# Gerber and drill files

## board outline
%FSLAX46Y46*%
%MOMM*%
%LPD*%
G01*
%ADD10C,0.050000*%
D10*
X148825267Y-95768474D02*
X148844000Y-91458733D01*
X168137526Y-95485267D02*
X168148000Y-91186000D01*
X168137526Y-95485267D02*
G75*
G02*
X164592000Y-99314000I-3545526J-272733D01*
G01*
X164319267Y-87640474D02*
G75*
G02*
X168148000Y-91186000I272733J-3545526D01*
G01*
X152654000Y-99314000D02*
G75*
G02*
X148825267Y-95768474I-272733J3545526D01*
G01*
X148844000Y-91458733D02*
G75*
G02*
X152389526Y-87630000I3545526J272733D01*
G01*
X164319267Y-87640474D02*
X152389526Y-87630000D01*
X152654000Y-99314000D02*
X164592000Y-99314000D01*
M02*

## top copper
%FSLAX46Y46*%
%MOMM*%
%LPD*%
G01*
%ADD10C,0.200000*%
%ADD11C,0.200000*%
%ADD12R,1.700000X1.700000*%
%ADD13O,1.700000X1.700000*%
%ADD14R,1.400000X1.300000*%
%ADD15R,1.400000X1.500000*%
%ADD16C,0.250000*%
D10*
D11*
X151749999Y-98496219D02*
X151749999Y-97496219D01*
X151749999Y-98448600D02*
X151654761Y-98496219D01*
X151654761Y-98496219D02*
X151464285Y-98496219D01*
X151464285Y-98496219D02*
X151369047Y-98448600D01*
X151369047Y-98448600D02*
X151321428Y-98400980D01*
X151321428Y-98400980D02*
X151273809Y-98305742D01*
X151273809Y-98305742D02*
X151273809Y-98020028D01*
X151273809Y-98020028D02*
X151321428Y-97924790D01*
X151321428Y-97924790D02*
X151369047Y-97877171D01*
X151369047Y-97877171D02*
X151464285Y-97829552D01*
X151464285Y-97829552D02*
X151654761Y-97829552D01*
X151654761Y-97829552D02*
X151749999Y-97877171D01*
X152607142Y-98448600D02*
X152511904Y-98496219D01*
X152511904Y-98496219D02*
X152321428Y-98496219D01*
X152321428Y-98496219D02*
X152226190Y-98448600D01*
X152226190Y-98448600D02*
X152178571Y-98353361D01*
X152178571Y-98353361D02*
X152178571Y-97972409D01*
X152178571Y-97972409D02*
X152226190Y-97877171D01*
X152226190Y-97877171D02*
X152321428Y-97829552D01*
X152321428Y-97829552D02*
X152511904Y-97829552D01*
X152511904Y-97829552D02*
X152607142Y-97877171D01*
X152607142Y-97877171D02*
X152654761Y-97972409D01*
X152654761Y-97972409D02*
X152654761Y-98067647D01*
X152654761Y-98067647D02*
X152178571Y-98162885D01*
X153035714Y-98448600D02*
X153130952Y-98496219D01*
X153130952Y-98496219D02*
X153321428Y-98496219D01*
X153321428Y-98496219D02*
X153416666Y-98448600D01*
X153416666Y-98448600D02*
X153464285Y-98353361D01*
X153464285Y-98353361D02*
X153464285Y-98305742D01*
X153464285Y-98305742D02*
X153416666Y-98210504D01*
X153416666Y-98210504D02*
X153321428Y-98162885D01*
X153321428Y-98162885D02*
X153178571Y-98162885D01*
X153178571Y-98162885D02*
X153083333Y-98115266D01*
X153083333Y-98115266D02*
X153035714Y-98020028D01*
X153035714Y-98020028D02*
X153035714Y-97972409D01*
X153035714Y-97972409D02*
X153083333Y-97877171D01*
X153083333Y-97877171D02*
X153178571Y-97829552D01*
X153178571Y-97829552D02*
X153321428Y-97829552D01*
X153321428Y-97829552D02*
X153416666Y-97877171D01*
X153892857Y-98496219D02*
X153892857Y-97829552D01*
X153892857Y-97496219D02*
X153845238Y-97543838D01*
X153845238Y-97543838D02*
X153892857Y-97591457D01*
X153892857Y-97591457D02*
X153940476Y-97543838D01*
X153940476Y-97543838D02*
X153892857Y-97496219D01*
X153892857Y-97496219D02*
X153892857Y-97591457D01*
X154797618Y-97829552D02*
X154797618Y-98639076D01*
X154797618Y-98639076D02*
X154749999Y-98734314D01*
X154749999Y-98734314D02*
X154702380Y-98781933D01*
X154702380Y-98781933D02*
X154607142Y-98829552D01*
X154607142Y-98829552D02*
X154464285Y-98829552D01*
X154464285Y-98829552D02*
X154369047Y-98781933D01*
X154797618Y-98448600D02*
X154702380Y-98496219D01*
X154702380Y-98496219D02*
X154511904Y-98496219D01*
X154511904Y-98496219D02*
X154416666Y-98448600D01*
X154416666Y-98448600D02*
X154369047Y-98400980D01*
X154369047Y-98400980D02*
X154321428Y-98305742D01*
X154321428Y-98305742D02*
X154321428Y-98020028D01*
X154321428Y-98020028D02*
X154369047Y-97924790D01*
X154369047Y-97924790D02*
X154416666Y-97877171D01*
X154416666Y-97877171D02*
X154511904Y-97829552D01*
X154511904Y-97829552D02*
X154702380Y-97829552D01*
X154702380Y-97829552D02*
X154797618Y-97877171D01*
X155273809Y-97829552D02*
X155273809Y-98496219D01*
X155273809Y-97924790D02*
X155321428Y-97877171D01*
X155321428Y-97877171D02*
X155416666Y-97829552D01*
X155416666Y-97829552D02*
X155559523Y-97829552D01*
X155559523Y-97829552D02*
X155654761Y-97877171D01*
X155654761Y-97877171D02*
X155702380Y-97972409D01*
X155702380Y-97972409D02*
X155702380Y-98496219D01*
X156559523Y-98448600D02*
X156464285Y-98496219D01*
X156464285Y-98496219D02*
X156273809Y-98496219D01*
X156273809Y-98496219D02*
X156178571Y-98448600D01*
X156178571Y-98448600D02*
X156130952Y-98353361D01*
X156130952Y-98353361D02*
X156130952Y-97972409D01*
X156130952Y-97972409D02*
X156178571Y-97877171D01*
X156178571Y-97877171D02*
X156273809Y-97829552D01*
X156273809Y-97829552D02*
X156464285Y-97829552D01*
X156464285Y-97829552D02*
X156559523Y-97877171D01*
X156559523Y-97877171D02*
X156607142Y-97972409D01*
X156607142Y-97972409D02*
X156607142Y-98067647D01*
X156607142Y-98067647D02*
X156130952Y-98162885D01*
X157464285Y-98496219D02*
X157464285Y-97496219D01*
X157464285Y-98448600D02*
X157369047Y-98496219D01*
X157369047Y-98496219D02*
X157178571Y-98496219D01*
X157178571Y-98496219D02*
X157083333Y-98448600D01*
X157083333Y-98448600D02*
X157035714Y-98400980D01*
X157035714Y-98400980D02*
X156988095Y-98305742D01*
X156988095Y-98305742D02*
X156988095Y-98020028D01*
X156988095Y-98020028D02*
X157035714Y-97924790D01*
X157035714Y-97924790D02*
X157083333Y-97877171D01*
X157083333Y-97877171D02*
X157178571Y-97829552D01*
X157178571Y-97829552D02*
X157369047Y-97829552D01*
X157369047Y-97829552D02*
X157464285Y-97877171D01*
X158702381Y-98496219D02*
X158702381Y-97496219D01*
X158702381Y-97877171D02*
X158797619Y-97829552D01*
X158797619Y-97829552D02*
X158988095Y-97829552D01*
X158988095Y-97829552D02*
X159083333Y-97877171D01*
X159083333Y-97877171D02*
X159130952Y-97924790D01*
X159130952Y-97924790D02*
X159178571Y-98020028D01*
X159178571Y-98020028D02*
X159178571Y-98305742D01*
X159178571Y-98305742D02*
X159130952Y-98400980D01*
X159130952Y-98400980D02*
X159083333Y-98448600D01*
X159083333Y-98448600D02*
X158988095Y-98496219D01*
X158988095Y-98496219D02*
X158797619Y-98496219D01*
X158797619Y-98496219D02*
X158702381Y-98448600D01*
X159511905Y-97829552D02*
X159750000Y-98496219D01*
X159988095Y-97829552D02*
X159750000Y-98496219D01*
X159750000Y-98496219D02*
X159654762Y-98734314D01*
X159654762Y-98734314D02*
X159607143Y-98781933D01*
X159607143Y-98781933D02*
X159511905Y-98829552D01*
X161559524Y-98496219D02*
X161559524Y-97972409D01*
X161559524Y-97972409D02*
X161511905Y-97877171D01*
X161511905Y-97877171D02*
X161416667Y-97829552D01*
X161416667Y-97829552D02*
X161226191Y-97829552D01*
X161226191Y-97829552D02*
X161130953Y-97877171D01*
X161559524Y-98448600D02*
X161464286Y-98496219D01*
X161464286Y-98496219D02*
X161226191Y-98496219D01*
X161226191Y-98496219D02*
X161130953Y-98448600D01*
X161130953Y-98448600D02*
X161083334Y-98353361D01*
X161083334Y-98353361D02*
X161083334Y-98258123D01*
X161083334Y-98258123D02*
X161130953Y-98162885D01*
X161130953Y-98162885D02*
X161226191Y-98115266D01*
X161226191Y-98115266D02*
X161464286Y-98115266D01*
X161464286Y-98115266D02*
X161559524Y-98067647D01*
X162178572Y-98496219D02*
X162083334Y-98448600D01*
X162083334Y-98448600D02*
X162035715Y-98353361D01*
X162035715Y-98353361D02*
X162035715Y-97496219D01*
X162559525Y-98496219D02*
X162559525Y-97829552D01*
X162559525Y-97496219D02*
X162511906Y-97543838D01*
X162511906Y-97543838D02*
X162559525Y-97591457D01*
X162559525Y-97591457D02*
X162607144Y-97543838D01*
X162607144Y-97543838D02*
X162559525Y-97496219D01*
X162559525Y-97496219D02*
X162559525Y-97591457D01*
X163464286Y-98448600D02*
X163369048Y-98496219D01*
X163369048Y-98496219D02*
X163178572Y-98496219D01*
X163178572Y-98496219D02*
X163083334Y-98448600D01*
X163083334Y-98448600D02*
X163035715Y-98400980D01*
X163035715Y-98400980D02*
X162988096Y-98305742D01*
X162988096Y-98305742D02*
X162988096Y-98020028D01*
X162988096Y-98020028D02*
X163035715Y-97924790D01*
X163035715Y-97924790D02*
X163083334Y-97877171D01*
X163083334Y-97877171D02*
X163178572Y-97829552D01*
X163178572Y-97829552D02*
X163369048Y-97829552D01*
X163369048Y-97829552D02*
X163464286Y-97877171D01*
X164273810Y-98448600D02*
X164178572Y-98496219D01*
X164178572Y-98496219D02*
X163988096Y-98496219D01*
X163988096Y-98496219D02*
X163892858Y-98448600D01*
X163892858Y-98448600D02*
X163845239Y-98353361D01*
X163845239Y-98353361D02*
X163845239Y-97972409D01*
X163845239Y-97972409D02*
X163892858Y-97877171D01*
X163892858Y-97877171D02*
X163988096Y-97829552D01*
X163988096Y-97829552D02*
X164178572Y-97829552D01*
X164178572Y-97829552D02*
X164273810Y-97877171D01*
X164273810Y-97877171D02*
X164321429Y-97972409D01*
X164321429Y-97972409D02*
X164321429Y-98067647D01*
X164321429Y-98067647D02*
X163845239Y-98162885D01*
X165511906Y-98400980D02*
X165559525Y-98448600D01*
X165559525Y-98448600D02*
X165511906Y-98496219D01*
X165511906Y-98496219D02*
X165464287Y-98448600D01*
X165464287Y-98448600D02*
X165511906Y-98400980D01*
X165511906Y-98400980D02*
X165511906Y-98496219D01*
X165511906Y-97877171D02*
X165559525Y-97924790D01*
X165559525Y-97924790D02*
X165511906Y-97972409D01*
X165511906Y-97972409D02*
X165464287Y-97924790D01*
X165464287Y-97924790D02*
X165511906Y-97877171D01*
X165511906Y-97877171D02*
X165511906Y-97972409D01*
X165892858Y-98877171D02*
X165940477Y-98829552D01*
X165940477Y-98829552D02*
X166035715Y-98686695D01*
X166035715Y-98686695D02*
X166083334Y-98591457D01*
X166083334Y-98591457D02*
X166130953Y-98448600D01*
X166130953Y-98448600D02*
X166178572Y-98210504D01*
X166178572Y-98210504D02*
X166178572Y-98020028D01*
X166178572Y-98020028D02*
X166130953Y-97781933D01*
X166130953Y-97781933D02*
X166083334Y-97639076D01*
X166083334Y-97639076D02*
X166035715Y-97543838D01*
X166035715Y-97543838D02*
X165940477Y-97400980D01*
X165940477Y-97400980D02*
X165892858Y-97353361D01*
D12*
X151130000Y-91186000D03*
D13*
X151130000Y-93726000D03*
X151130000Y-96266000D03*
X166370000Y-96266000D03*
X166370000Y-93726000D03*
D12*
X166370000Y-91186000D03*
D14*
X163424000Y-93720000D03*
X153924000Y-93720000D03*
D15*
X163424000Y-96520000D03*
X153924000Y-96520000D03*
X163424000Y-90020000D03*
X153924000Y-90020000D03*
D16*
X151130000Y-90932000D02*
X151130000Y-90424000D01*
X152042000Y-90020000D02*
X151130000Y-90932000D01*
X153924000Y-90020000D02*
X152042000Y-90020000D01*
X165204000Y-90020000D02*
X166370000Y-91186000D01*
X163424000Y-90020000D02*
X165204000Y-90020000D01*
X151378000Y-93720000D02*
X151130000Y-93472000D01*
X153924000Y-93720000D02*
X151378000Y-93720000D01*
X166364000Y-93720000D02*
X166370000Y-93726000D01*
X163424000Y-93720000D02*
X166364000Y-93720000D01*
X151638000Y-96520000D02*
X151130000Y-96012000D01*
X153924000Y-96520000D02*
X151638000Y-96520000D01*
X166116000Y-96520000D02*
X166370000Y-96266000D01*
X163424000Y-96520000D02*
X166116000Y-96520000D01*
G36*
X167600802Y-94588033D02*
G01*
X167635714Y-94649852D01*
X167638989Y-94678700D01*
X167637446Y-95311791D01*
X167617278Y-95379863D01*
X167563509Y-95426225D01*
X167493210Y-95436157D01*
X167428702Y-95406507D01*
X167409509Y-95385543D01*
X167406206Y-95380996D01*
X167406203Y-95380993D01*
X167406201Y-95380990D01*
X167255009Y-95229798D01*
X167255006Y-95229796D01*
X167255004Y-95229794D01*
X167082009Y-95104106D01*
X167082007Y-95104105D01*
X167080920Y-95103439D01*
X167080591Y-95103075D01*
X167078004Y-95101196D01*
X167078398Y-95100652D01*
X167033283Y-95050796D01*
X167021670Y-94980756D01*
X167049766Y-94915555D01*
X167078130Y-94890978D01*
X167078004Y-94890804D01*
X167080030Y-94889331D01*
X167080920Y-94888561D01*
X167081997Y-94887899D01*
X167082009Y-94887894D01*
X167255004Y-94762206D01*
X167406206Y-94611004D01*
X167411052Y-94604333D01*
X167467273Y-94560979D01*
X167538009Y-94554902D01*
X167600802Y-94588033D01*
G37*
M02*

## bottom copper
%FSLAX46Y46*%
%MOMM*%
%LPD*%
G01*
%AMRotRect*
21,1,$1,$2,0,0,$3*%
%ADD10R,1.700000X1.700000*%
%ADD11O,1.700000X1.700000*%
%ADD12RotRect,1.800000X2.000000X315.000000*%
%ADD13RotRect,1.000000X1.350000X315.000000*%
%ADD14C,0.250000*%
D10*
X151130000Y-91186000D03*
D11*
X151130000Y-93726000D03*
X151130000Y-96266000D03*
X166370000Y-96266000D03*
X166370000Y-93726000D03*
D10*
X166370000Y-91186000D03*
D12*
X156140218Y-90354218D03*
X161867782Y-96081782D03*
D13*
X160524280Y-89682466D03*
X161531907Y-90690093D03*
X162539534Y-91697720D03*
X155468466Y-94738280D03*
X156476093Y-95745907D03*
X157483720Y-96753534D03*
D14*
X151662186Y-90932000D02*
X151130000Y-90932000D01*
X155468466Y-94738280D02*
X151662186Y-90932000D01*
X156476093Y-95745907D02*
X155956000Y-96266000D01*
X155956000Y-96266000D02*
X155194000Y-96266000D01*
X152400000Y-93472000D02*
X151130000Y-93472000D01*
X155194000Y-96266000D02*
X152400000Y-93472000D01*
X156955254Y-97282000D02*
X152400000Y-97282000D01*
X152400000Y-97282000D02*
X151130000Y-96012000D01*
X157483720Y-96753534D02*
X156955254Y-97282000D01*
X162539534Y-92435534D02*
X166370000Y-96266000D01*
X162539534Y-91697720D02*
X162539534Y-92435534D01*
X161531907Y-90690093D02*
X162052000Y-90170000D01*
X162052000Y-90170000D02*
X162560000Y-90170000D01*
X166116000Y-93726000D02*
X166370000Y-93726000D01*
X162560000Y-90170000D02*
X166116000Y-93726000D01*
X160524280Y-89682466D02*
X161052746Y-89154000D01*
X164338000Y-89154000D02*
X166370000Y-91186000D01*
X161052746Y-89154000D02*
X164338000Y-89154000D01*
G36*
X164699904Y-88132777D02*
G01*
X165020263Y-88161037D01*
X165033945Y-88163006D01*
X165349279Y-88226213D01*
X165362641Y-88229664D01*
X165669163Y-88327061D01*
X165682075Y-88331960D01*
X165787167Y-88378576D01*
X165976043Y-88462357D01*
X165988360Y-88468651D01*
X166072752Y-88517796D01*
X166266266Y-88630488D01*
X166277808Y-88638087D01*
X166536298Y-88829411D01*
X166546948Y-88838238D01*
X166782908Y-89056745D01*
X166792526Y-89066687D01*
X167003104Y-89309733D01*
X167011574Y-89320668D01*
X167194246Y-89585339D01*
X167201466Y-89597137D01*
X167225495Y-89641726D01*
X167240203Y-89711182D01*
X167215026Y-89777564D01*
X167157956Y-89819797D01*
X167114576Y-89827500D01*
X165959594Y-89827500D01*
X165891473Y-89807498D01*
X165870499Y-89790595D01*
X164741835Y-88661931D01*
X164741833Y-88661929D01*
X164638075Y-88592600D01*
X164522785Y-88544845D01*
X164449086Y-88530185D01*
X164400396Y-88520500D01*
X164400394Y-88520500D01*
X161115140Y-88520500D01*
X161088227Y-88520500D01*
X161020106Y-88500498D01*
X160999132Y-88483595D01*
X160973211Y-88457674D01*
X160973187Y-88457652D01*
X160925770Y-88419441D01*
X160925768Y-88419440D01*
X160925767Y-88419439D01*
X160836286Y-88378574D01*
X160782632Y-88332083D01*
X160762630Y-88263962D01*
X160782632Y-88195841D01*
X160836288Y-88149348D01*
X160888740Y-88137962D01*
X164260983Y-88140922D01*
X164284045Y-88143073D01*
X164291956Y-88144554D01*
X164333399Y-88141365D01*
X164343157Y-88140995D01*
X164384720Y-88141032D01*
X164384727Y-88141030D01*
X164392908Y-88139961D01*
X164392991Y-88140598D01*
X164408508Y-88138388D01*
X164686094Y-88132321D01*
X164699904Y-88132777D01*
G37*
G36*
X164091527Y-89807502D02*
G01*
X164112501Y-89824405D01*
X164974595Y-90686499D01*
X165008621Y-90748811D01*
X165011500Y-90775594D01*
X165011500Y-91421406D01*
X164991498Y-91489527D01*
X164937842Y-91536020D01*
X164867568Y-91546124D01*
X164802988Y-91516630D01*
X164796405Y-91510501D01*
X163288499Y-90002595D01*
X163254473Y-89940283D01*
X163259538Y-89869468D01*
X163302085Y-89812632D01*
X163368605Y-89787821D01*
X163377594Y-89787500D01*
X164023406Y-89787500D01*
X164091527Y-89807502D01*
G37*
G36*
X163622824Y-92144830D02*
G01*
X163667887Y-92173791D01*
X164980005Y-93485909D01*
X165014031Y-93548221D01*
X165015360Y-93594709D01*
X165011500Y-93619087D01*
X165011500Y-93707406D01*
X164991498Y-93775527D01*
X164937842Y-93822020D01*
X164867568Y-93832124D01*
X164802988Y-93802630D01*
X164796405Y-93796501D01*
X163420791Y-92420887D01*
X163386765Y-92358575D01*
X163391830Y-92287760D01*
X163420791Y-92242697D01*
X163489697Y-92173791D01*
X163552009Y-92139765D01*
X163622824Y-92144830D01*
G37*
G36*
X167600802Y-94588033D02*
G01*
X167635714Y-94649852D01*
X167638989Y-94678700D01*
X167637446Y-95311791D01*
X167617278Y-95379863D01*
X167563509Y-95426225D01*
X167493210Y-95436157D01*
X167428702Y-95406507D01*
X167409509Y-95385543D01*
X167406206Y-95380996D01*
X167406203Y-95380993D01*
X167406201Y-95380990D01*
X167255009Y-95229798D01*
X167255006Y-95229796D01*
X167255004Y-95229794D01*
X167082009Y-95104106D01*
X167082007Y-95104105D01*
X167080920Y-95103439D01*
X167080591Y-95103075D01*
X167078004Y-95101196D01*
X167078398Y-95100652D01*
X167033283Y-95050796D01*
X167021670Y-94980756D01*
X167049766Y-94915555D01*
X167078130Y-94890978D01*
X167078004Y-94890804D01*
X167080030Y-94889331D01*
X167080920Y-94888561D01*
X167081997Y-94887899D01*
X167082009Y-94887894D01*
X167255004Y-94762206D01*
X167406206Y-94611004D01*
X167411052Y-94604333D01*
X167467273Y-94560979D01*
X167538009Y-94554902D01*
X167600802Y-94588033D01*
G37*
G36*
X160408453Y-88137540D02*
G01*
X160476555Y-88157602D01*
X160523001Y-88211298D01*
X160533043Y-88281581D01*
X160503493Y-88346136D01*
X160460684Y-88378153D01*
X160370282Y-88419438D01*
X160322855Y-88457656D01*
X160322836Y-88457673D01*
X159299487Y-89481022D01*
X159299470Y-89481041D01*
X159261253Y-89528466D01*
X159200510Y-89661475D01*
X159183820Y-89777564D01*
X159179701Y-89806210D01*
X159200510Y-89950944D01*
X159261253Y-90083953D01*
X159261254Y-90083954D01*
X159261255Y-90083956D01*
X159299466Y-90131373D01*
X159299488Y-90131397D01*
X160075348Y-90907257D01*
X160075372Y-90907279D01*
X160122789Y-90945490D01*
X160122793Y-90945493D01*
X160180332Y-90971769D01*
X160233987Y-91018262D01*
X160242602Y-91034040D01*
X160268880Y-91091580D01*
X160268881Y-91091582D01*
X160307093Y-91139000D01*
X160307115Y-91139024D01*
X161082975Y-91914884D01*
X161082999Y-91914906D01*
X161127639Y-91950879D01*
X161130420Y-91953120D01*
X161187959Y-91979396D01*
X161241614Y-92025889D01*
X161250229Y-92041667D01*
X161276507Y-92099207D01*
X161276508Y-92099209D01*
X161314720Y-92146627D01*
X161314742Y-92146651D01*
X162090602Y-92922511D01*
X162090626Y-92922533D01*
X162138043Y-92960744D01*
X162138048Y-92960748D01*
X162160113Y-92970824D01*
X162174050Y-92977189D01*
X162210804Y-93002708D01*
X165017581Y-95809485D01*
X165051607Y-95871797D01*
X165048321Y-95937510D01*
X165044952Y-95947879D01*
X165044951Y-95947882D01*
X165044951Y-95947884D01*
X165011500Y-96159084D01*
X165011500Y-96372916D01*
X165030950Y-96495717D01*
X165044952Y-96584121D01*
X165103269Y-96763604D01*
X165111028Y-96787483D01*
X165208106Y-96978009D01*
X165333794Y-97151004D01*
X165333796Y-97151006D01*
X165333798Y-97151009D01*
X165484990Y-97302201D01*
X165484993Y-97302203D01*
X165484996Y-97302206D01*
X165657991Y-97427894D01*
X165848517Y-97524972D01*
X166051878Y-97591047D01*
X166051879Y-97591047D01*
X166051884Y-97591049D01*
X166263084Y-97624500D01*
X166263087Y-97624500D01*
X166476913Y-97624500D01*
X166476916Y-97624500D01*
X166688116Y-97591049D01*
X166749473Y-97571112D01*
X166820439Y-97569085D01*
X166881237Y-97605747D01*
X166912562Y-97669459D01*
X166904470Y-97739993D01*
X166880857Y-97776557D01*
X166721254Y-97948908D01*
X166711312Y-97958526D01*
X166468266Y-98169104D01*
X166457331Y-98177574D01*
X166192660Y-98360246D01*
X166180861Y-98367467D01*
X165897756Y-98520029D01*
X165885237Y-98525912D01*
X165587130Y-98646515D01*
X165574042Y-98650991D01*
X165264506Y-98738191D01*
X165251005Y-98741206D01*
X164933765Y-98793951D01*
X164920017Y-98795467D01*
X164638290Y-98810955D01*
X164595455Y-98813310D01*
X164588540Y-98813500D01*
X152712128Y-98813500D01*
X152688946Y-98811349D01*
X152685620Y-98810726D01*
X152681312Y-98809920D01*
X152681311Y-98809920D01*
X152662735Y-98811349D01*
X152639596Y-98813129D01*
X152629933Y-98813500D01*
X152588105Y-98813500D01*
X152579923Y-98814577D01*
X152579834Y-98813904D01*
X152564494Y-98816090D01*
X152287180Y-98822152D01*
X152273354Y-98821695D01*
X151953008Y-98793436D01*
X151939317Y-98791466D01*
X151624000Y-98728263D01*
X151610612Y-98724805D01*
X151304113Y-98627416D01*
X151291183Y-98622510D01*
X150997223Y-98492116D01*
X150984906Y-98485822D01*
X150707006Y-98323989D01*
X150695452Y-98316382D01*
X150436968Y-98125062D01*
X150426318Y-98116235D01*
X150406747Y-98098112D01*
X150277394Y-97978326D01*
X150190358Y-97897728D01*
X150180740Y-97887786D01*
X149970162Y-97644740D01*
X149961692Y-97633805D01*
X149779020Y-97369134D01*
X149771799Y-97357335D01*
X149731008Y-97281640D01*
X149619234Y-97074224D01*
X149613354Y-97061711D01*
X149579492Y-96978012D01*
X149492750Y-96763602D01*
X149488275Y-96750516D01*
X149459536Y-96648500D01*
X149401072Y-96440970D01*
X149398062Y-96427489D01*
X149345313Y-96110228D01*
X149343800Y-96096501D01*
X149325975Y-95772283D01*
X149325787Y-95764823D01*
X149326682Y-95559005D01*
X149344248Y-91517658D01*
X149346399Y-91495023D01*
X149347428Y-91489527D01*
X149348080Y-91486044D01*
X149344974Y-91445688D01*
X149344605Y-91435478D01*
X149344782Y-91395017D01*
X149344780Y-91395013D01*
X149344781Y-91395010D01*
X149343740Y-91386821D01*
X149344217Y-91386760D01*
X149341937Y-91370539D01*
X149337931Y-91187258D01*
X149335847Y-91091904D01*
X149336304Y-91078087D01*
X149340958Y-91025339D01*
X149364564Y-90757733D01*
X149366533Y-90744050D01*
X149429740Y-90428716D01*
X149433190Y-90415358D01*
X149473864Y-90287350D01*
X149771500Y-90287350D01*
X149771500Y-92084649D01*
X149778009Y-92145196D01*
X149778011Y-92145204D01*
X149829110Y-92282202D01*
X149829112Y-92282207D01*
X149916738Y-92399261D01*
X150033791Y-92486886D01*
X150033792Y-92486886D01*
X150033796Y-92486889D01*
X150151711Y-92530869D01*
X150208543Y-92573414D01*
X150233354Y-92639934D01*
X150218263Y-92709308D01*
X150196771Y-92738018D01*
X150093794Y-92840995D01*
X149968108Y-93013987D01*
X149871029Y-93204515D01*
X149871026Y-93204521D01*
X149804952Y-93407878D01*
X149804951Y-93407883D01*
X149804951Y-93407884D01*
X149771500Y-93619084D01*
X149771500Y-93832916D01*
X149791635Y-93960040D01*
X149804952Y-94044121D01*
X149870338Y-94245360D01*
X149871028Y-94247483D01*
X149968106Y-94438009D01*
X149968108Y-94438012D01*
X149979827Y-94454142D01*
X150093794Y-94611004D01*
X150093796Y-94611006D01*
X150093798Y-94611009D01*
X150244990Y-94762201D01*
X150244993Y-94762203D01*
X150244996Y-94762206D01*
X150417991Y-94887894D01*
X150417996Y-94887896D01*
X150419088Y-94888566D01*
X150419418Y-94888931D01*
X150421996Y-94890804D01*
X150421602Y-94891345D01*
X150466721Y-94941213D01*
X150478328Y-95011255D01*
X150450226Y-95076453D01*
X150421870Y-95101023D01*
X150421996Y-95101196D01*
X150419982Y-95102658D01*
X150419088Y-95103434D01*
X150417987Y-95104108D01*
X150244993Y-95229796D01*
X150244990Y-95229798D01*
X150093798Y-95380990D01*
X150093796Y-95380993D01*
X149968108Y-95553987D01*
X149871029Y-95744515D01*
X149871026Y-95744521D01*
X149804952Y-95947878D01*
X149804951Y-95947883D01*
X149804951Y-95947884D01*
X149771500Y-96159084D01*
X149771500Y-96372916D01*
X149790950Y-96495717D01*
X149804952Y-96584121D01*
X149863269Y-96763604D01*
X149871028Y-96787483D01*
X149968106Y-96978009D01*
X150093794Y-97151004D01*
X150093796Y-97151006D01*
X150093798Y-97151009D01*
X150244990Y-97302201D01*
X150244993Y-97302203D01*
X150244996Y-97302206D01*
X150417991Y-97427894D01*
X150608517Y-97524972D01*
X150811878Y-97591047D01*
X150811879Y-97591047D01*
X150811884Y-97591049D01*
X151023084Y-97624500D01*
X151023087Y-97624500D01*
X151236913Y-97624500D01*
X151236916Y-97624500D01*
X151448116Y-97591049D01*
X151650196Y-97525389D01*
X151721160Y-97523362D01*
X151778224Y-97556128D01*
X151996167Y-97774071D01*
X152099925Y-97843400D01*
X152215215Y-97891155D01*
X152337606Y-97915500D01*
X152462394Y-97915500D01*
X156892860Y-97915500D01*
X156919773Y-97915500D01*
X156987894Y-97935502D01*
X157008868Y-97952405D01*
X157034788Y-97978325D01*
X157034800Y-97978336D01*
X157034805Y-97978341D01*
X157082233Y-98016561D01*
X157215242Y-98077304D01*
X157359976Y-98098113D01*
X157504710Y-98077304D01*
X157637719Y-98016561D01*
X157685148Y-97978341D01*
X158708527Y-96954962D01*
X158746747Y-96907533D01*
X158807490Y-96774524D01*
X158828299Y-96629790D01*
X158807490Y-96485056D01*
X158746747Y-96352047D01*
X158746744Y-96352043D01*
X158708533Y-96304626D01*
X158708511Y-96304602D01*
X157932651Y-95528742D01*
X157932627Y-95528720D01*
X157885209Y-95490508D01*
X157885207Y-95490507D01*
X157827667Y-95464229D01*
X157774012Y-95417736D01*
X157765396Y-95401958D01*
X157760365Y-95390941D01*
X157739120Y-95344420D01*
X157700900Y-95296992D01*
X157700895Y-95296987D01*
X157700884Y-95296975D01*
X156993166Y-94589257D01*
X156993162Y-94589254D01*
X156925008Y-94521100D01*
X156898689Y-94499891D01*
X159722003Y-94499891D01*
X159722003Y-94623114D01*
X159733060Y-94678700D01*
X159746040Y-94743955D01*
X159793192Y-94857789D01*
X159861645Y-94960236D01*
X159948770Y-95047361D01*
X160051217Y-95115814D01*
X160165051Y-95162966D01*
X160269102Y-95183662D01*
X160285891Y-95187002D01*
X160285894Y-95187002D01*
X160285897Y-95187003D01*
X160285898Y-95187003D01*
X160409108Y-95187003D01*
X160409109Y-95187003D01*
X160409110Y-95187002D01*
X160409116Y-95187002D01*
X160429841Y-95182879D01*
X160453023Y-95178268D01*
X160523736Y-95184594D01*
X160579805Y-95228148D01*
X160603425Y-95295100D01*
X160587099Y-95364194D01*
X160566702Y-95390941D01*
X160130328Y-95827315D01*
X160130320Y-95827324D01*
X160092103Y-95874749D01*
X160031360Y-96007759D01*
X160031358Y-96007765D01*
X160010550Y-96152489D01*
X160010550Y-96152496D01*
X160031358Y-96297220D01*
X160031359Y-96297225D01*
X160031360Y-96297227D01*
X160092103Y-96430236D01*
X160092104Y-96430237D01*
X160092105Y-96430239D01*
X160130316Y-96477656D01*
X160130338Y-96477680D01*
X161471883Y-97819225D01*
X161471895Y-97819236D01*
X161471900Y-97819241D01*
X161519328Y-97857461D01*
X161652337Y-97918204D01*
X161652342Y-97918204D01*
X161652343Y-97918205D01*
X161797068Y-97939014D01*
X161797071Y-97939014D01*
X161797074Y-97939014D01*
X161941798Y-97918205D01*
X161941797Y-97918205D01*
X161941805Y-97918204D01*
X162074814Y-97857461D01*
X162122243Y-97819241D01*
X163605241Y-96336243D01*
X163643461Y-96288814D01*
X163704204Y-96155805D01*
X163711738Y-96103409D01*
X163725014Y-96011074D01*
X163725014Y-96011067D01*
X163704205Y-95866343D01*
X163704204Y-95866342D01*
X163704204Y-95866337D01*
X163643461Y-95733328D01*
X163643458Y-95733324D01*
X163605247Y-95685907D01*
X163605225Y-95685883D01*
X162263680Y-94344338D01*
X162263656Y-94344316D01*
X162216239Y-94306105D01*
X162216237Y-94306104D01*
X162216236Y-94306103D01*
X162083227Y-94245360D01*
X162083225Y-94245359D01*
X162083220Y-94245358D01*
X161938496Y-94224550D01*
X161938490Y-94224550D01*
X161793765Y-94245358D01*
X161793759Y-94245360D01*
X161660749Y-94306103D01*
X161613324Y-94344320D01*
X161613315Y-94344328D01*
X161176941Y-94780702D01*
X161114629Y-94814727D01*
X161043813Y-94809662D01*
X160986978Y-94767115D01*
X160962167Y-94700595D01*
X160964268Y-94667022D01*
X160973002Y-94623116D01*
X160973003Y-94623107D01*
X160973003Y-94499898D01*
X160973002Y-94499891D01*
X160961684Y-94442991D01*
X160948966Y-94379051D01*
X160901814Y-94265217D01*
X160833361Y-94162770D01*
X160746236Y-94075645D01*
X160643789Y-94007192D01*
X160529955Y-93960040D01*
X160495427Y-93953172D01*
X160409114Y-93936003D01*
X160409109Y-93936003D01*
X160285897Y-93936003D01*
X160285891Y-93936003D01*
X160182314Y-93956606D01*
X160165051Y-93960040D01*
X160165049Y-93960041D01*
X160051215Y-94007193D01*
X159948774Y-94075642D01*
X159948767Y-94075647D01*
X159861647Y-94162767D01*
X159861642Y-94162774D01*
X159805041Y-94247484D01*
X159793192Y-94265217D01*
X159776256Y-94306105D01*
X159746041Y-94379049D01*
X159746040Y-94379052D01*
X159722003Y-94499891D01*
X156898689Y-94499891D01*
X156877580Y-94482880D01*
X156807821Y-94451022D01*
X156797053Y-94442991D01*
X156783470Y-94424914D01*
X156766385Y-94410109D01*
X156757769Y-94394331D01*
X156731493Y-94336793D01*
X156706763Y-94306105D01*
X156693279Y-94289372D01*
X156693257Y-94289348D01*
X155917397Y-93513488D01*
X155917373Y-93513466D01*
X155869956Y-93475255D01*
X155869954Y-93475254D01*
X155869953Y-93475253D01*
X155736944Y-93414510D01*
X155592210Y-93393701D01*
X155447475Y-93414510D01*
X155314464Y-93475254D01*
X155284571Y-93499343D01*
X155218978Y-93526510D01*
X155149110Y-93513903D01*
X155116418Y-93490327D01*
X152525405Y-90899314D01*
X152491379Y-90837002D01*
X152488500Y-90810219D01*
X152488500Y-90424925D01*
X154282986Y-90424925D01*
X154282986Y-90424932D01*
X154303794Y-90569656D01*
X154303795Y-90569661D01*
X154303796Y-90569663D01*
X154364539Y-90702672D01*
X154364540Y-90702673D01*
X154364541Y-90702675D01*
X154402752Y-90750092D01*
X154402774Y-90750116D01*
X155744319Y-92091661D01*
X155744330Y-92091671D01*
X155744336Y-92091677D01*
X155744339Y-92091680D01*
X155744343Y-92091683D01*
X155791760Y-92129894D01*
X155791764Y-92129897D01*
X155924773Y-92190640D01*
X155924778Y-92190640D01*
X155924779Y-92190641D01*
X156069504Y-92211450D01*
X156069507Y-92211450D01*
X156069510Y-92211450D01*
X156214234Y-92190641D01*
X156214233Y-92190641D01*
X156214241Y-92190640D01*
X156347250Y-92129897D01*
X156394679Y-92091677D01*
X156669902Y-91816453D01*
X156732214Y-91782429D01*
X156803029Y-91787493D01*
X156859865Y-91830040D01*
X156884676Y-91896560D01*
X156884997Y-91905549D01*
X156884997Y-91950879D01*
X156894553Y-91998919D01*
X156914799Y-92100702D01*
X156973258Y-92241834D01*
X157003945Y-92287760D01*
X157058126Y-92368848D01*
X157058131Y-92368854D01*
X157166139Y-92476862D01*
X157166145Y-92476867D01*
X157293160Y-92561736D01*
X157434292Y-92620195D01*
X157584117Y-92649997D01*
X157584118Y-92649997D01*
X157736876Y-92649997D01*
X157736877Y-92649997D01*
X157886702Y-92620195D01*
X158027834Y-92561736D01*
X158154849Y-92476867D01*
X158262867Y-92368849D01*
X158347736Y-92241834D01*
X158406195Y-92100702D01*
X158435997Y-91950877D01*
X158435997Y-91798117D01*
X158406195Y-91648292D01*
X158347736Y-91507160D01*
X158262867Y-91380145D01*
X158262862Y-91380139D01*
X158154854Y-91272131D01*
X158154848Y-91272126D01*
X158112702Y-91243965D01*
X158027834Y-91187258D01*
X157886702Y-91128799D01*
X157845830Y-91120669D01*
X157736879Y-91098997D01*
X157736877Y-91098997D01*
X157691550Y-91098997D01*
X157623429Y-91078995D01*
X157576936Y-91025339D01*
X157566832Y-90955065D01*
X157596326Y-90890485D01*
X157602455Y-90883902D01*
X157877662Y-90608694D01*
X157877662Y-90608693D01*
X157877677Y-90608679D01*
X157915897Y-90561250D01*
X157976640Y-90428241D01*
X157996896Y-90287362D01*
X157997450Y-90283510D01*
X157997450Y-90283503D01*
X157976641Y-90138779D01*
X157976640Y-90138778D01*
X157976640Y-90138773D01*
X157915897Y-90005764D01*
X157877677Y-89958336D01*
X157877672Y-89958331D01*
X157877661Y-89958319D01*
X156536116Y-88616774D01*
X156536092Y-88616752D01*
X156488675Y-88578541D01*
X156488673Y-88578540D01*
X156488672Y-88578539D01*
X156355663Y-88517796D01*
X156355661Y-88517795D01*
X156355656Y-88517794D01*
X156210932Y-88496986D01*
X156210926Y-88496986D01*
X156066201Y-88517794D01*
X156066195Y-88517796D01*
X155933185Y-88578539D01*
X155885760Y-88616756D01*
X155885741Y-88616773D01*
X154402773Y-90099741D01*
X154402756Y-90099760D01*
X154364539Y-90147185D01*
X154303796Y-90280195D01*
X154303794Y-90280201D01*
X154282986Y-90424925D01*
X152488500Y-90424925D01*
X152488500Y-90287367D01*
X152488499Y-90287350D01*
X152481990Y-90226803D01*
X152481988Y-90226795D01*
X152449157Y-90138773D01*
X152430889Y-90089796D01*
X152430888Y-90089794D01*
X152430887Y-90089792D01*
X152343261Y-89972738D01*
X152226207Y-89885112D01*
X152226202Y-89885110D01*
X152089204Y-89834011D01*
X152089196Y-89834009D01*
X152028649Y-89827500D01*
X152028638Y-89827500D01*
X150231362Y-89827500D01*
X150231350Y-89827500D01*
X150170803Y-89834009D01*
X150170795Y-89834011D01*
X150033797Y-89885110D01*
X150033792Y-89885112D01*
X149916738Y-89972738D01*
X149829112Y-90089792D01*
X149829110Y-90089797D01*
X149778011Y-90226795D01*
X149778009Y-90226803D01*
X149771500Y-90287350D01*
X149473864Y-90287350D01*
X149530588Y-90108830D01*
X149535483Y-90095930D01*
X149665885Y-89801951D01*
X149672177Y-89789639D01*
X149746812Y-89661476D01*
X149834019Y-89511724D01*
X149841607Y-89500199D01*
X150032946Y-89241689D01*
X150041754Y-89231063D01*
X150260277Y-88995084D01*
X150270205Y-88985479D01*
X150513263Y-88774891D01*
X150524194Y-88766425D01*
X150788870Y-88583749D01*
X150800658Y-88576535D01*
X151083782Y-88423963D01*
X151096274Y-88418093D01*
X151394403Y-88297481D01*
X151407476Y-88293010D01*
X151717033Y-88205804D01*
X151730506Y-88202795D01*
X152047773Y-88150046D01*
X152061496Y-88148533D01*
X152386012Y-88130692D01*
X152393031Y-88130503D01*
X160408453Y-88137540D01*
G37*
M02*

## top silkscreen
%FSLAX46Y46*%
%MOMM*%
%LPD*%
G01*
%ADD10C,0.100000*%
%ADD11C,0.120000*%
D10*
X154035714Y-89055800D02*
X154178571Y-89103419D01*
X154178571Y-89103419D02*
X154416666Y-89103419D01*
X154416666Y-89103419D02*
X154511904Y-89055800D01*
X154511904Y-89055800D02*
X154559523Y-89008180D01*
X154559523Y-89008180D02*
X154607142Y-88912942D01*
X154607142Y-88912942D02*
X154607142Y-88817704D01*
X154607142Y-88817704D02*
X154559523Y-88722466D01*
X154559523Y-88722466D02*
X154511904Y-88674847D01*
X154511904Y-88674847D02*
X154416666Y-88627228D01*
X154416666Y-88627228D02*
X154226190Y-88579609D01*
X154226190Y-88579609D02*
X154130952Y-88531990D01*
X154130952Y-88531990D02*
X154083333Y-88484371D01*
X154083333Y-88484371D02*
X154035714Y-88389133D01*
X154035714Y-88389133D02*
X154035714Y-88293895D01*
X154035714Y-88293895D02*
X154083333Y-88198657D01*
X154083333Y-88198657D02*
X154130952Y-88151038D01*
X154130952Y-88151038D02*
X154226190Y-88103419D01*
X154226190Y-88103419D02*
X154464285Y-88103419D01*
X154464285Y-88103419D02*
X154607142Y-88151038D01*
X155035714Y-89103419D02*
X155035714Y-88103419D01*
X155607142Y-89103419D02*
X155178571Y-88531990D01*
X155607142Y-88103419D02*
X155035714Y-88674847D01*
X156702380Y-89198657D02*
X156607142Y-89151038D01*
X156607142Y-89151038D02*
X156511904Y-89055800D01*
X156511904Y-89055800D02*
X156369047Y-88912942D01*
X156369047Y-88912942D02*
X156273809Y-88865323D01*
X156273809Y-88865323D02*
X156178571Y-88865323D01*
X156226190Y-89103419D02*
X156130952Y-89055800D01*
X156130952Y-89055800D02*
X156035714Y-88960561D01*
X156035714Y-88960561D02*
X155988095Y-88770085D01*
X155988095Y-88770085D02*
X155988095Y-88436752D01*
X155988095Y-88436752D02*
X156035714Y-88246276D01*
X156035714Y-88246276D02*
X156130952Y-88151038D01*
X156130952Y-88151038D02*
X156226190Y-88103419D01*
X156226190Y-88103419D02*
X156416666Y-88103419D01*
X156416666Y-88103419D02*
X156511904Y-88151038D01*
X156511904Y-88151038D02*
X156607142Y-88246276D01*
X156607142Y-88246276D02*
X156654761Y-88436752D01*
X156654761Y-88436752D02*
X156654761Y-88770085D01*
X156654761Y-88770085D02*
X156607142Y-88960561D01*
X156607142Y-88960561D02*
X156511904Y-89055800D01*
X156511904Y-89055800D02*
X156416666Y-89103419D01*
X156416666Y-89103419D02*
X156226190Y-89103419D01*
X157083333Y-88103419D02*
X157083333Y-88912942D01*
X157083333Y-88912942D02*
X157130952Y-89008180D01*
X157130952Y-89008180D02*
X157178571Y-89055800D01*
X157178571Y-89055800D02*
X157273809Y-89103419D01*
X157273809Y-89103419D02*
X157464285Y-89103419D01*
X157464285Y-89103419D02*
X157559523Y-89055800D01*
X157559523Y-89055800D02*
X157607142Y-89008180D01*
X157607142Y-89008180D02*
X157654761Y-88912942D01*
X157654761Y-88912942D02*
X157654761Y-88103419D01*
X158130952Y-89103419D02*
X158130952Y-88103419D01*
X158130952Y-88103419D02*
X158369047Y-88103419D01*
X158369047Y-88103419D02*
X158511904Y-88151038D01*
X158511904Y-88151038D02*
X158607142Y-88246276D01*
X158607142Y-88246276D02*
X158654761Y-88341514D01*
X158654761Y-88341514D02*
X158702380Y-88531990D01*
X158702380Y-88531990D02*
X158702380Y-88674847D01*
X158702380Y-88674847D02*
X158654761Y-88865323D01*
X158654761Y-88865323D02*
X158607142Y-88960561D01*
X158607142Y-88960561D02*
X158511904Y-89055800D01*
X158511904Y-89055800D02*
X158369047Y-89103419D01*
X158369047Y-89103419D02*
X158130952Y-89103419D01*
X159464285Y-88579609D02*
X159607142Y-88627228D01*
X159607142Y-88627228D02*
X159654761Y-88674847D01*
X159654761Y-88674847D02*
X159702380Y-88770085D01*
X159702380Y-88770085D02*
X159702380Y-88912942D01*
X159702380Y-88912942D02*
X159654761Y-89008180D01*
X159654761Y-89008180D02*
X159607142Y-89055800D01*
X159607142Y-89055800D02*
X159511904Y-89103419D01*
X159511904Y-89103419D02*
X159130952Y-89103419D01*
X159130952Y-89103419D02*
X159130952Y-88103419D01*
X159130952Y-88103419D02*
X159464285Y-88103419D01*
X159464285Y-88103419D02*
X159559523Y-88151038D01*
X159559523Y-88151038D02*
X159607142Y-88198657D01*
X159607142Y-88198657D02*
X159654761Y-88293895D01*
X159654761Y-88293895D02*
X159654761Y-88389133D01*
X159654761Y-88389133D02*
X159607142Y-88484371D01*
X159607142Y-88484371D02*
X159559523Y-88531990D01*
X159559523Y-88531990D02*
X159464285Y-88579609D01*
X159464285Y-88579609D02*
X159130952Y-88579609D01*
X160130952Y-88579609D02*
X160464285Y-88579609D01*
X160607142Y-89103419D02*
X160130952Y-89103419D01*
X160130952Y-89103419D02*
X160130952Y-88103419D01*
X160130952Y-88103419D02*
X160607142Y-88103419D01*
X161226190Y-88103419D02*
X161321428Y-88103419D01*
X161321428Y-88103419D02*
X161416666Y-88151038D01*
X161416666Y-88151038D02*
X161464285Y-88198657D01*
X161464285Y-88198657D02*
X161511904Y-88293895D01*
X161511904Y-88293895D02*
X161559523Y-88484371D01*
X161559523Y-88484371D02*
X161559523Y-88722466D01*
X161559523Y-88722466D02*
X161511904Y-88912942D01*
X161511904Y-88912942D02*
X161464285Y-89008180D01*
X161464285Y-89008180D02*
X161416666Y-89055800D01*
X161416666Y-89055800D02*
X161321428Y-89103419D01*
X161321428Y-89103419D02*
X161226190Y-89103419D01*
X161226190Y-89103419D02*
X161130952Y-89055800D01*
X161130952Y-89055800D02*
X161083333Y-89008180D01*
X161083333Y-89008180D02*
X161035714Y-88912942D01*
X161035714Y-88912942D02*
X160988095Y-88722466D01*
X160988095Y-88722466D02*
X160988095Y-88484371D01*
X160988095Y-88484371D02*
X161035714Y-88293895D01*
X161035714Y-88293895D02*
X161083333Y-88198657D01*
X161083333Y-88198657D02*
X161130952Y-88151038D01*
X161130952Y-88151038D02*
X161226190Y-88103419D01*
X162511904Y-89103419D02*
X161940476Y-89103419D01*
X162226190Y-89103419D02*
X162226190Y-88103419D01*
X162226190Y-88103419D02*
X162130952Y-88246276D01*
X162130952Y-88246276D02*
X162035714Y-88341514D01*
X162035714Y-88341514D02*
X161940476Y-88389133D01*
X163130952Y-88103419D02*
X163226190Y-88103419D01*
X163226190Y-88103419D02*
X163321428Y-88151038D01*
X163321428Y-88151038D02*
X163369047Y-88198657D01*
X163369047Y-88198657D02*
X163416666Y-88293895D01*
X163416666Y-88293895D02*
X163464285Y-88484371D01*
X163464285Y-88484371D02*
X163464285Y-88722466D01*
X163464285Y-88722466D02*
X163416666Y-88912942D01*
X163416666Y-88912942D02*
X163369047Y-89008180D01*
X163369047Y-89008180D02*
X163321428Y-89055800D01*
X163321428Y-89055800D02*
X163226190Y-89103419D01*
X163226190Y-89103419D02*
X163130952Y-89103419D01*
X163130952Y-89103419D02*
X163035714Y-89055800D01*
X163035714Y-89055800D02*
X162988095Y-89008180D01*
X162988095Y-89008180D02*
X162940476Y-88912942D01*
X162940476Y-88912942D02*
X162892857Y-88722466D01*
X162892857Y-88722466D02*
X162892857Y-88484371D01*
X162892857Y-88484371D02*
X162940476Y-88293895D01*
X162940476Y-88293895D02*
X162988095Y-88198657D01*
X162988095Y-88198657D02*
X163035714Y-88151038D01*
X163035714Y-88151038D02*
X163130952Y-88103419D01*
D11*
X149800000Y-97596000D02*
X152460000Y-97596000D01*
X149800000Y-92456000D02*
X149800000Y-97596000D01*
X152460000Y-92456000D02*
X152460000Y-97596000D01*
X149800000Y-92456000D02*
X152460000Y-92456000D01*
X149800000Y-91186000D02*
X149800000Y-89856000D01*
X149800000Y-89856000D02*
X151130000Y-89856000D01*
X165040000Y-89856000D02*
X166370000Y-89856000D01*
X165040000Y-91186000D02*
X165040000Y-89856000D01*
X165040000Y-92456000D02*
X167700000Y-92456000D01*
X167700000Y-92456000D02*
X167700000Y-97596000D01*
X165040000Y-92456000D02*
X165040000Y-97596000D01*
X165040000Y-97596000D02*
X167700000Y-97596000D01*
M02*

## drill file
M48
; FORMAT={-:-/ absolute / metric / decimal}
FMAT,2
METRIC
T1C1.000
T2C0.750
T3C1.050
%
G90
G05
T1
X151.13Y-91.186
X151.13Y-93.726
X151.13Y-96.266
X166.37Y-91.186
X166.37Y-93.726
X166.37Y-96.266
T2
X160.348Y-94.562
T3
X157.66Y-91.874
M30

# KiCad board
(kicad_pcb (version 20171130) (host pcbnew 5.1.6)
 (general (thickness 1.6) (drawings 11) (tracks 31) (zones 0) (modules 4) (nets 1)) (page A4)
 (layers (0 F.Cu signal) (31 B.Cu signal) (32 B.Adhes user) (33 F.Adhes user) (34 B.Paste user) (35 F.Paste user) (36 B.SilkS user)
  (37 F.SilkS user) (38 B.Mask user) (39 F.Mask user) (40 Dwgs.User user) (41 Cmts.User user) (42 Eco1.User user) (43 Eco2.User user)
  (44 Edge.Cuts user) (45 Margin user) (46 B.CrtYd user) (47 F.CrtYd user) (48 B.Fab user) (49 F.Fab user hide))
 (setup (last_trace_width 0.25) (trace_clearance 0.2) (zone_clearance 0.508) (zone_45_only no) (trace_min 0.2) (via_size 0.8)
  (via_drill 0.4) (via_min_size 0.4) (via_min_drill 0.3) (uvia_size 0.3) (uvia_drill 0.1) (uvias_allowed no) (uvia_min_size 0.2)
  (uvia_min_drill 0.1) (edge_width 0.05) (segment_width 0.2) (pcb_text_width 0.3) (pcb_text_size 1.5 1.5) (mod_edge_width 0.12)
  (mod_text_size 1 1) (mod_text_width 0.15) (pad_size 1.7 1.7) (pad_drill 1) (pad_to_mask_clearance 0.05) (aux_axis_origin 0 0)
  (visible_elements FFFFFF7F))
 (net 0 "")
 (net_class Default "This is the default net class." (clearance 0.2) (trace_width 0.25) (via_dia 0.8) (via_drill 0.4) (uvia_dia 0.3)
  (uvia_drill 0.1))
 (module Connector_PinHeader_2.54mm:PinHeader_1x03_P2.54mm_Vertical (layer F.Cu) (at 151.13 91.186)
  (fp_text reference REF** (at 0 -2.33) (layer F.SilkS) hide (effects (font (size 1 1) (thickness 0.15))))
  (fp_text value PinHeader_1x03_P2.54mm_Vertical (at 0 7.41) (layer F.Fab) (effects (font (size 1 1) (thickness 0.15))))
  (fp_line (start -1.33 6.41) (end 1.33 6.41) (layer F.SilkS) (width 0.12))
  (fp_line (start -1.33 1.27) (end -1.33 6.41) (layer F.SilkS) (width 0.12))
  (fp_line (start 1.33 1.27) (end 1.33 6.41) (layer F.SilkS) (width 0.12))
  (fp_line (start -1.33 1.27) (end 1.33 1.27) (layer F.SilkS) (width 0.12))
  (fp_line (start -1.33 0) (end -1.33 -1.33) (layer F.SilkS) (width 0.12))
  (fp_line (start -1.33 -1.33) (end 0 -1.33) (layer F.SilkS) (width 0.12))
  (pad 1 thru_hole rect (at 0 0) (size 1.7 1.7) (drill 1) (layers *.Cu *.Mask))
  (pad 2 thru_hole oval (at 0 2.54) (size 1.7 1.7) (drill 1) (layers *.Cu *.Mask))
  (pad 3 thru_hole oval (at 0 5.08) (size 1.7 1.7) (drill 1) (layers *.Cu *.Mask)))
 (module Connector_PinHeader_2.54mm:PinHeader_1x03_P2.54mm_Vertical (layer F.Cu) (at 166.37 91.186)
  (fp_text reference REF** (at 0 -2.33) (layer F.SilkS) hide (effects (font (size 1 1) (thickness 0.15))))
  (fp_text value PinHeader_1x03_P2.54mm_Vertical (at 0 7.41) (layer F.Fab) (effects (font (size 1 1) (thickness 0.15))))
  (fp_line (start -1.33 -1.33) (end 0 -1.33) (layer F.SilkS) (width 0.12))
  (fp_line (start -1.33 0) (end -1.33 -1.33) (layer F.SilkS) (width 0.12))
  (fp_line (start -1.33 1.27) (end 1.33 1.27) (layer F.SilkS) (width 0.12))
  (fp_line (start 1.33 1.27) (end 1.33 6.41) (layer F.SilkS) (width 0.12))
  (fp_line (start -1.33 1.27) (end -1.33 6.41) (layer F.SilkS) (width 0.12))
  (fp_line (start -1.33 6.41) (end 1.33 6.41) (layer F.SilkS) (width 0.12))
  (pad 3 thru_hole oval (at 0 5.08) (size 1.7 1.7) (drill 1) (layers *.Cu *.Mask))
  (pad 2 thru_hole oval (at 0 2.54) (size 1.7 1.7) (drill 1) (layers *.Cu *.Mask))
  (pad 1 thru_hole rect (at 0 0) (size 1.7 1.7) (drill 1) (layers *.Cu *.Mask)))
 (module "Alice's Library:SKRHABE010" (layer B.Cu) (at 159.004 93.218 45)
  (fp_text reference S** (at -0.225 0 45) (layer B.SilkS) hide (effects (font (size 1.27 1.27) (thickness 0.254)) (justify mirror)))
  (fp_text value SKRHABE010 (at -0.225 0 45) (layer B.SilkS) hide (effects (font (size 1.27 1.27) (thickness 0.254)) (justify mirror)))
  (pad GB2 np_thru_hole circle (at 0 -1.9 45) (size 1.05 0) (drill 1.05) (layers *.Cu *.Mask))
  (pad GB1 np_thru_hole circle (at 0 1.9 45) (size 0.75 0) (drill 0.75) (layers *.Cu *.Mask))
  (pad 8 smd rect (at 0 -4.05 315) (size 1.8 2) (layers B.Cu B.Paste B.Mask))
  (pad 7 smd rect (at 0 4.05 315) (size 1.8 2) (layers B.Cu B.Paste B.Mask))
  (pad 6 smd rect (at 3.575 -1.425 315) (size 1 1.35) (layers B.Cu B.Paste B.Mask))
  (pad 5 smd rect (at 3.575 0 315) (size 1 1.35) (layers B.Cu B.Paste B.Mask))
  (pad 4 smd rect (at 3.575 1.425 315) (size 1 1.35) (layers B.Cu B.Paste B.Mask))
  (pad 3 smd rect (at -3.575 -1.425 315) (size 1 1.35) (layers B.Cu B.Paste B.Mask))
  (pad 2 smd rect (at -3.575 0 315) (size 1 1.35) (layers B.Cu B.Paste B.Mask))
  (pad 1 smd rect (at -3.575 1.425 315) (size 1 1.35) (layers B.Cu B.Paste B.Mask)))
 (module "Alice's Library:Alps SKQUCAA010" (layer F.Cu) (at 153.924 90.02)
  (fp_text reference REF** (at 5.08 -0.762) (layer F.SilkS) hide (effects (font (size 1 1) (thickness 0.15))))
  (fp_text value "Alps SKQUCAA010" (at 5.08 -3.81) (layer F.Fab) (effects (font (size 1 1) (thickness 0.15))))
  (pad 5 smd rect (at 9.5 3.7) (size 1.4 1.3) (layers F.Cu F.Paste F.Mask))
  (pad 2 smd rect (at 0 3.7) (size 1.4 1.3) (layers F.Cu F.Paste F.Mask))
  (pad 4 smd rect (at 9.5 6.5) (size 1.4 1.5) (layers F.Cu F.Paste F.Mask))
  (pad 3 smd rect (at 0 6.5) (size 1.4 1.5) (layers F.Cu F.Paste F.Mask))
  (pad 6 smd rect (at 9.5 0) (size 1.4 1.5) (layers F.Cu F.Paste F.Mask))
  (pad 1 smd rect (at 0 0) (size 1.4 1.5) (layers F.Cu F.Paste F.Mask)))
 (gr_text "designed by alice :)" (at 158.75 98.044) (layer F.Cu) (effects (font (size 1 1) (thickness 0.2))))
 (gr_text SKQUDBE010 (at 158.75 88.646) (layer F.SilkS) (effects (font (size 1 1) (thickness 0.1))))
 (gr_line (start 148.825267 95.768474) (end 148.844 91.458733) (layer Edge.Cuts) (width 0.05))
 (gr_line (start 168.137526 95.485267) (end 168.148 91.186) (layer Edge.Cuts) (width 0.05))
 (gr_arc (start 164.592 95.758) (end 164.592 99.314) (angle -94.39870535) (layer Edge.Cuts) (width 0.05))
 (gr_arc (start 164.592 91.186) (end 168.148 91.186) (angle -94.39870535) (layer Edge.Cuts) (width 0.05))
 (gr_arc (start 152.381267 95.768474) (end 148.825267 95.768474) (angle -94.39870535) (layer Edge.Cuts) (width 0.05))
 (gr_arc (start 152.389526 91.186) (end 152.389526 87.63) (angle -94.39870535) (layer Edge.Cuts) (width 0.05))
 (gr_line (start 164.319267 87.640474) (end 152.389526 87.63) (layer Edge.Cuts) (width 0.05))
 (gr_line (start 152.654 99.314) (end 164.592 99.314) (layer Edge.Cuts) (width 0.05))
 (segment (start 151.13 90.932) (end 151.13 90.424) (width 0.25) (layer F.Cu) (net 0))
 (segment (start 152.042 90.02) (end 151.13 90.932) (width 0.25) (layer F.Cu) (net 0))
 (segment (start 153.924 90.02) (end 152.042 90.02) (width 0.25) (layer F.Cu) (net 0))
 (segment (start 165.204 90.02) (end 166.37 91.186) (width 0.25) (layer F.Cu) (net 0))
 (segment (start 163.424 90.02) (end 165.204 90.02) (width 0.25) (layer F.Cu) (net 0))
 (segment (start 151.378 93.72) (end 151.13 93.472) (width 0.25) (layer F.Cu) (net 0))
 (segment (start 153.924 93.72) (end 151.378 93.72) (width 0.25) (layer F.Cu) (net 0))
 (segment (start 166.364 93.72) (end 166.37 93.726) (width 0.25) (layer F.Cu) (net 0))
 (segment (start 163.424 93.72) (end 166.364 93.72) (width 0.25) (layer F.Cu) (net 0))
 (segment (start 151.638 96.52) (end 151.13 96.012) (width 0.25) (layer F.Cu) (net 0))
 (segment (start 153.924 96.52) (end 151.638 96.52) (width 0.25) (layer F.Cu) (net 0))
 (segment (start 166.116 96.52) (end 166.37 96.266) (width 0.25) (layer F.Cu) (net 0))
 (segment (start 163.424 96.52) (end 166.116 96.52) (width 0.25) (layer F.Cu) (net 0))
 (segment (start 151.662186 90.932) (end 151.13 90.932) (width 0.25) (layer B.Cu) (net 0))
 (segment (start 155.468466 94.73828) (end 151.662186 90.932) (width 0.25) (layer B.Cu) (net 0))
 (segment (start 156.476093 95.745907) (end 155.956 96.266) (width 0.25) (layer B.Cu) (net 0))
 (segment (start 155.956 96.266) (end 155.194 96.266) (width 0.25) (layer B.Cu) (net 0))
 (segment (start 152.4 93.472) (end 151.13 93.472) (width 0.25) (layer B.Cu) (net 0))
 (segment (start 155.194 96.266) (end 152.4 93.472) (width 0.25) (layer B.Cu) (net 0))
 (segment (start 156.955254 97.282) (end 152.4 97.282) (width 0.25) (layer B.Cu) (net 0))
 (segment (start 152.4 97.282) (end 151.13 96.012) (width 0.25) (layer B.Cu) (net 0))
 (segment (start 157.48372 96.753534) (end 156.955254 97.282) (width 0.25) (layer B.Cu) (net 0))
 (segment (start 162.539534 92.435534) (end 166.37 96.266) (width 0.25) (layer B.Cu) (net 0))
 (segment (start 162.539534 91.69772) (end 162.539534 92.435534) (width 0.25) (layer B.Cu) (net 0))
 (segment (start 161.531907 90.690093) (end 162.052 90.17) (width 0.25) (layer B.Cu) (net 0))
 (segment (start 162.052 90.17) (end 162.56 90.17) (width 0.25) (layer B.Cu) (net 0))
 (segment (start 166.116 93.726) (end 166.37 93.726) (width 0.25) (layer B.Cu) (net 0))
 (segment (start 162.56 90.17) (end 166.116 93.726) (width 0.25) (layer B.Cu) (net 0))
 (segment (start 160.52428 89.682466) (end 161.052746 89.154) (width 0.25) (layer B.Cu) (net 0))
 (segment (start 164.338 89.154) (end 166.37 91.186) (width 0.25) (layer B.Cu) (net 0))
 (segment (start 161.052746 89.154) (end 164.338 89.154) (width 0.25) (layer B.Cu) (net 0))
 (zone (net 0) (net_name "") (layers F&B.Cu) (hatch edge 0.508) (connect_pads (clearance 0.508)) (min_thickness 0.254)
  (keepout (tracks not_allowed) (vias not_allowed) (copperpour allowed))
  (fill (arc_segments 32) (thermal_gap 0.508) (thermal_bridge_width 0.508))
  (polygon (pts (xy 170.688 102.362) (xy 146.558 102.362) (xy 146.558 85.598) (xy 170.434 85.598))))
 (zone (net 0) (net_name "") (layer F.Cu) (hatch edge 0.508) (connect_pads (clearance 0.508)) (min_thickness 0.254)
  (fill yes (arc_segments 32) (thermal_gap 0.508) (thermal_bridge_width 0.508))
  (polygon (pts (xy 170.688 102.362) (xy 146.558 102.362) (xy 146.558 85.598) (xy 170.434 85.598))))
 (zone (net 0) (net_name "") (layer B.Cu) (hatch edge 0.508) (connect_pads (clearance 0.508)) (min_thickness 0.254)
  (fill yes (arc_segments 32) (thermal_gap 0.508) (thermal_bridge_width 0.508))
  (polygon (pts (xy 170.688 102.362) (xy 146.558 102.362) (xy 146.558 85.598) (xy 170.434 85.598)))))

